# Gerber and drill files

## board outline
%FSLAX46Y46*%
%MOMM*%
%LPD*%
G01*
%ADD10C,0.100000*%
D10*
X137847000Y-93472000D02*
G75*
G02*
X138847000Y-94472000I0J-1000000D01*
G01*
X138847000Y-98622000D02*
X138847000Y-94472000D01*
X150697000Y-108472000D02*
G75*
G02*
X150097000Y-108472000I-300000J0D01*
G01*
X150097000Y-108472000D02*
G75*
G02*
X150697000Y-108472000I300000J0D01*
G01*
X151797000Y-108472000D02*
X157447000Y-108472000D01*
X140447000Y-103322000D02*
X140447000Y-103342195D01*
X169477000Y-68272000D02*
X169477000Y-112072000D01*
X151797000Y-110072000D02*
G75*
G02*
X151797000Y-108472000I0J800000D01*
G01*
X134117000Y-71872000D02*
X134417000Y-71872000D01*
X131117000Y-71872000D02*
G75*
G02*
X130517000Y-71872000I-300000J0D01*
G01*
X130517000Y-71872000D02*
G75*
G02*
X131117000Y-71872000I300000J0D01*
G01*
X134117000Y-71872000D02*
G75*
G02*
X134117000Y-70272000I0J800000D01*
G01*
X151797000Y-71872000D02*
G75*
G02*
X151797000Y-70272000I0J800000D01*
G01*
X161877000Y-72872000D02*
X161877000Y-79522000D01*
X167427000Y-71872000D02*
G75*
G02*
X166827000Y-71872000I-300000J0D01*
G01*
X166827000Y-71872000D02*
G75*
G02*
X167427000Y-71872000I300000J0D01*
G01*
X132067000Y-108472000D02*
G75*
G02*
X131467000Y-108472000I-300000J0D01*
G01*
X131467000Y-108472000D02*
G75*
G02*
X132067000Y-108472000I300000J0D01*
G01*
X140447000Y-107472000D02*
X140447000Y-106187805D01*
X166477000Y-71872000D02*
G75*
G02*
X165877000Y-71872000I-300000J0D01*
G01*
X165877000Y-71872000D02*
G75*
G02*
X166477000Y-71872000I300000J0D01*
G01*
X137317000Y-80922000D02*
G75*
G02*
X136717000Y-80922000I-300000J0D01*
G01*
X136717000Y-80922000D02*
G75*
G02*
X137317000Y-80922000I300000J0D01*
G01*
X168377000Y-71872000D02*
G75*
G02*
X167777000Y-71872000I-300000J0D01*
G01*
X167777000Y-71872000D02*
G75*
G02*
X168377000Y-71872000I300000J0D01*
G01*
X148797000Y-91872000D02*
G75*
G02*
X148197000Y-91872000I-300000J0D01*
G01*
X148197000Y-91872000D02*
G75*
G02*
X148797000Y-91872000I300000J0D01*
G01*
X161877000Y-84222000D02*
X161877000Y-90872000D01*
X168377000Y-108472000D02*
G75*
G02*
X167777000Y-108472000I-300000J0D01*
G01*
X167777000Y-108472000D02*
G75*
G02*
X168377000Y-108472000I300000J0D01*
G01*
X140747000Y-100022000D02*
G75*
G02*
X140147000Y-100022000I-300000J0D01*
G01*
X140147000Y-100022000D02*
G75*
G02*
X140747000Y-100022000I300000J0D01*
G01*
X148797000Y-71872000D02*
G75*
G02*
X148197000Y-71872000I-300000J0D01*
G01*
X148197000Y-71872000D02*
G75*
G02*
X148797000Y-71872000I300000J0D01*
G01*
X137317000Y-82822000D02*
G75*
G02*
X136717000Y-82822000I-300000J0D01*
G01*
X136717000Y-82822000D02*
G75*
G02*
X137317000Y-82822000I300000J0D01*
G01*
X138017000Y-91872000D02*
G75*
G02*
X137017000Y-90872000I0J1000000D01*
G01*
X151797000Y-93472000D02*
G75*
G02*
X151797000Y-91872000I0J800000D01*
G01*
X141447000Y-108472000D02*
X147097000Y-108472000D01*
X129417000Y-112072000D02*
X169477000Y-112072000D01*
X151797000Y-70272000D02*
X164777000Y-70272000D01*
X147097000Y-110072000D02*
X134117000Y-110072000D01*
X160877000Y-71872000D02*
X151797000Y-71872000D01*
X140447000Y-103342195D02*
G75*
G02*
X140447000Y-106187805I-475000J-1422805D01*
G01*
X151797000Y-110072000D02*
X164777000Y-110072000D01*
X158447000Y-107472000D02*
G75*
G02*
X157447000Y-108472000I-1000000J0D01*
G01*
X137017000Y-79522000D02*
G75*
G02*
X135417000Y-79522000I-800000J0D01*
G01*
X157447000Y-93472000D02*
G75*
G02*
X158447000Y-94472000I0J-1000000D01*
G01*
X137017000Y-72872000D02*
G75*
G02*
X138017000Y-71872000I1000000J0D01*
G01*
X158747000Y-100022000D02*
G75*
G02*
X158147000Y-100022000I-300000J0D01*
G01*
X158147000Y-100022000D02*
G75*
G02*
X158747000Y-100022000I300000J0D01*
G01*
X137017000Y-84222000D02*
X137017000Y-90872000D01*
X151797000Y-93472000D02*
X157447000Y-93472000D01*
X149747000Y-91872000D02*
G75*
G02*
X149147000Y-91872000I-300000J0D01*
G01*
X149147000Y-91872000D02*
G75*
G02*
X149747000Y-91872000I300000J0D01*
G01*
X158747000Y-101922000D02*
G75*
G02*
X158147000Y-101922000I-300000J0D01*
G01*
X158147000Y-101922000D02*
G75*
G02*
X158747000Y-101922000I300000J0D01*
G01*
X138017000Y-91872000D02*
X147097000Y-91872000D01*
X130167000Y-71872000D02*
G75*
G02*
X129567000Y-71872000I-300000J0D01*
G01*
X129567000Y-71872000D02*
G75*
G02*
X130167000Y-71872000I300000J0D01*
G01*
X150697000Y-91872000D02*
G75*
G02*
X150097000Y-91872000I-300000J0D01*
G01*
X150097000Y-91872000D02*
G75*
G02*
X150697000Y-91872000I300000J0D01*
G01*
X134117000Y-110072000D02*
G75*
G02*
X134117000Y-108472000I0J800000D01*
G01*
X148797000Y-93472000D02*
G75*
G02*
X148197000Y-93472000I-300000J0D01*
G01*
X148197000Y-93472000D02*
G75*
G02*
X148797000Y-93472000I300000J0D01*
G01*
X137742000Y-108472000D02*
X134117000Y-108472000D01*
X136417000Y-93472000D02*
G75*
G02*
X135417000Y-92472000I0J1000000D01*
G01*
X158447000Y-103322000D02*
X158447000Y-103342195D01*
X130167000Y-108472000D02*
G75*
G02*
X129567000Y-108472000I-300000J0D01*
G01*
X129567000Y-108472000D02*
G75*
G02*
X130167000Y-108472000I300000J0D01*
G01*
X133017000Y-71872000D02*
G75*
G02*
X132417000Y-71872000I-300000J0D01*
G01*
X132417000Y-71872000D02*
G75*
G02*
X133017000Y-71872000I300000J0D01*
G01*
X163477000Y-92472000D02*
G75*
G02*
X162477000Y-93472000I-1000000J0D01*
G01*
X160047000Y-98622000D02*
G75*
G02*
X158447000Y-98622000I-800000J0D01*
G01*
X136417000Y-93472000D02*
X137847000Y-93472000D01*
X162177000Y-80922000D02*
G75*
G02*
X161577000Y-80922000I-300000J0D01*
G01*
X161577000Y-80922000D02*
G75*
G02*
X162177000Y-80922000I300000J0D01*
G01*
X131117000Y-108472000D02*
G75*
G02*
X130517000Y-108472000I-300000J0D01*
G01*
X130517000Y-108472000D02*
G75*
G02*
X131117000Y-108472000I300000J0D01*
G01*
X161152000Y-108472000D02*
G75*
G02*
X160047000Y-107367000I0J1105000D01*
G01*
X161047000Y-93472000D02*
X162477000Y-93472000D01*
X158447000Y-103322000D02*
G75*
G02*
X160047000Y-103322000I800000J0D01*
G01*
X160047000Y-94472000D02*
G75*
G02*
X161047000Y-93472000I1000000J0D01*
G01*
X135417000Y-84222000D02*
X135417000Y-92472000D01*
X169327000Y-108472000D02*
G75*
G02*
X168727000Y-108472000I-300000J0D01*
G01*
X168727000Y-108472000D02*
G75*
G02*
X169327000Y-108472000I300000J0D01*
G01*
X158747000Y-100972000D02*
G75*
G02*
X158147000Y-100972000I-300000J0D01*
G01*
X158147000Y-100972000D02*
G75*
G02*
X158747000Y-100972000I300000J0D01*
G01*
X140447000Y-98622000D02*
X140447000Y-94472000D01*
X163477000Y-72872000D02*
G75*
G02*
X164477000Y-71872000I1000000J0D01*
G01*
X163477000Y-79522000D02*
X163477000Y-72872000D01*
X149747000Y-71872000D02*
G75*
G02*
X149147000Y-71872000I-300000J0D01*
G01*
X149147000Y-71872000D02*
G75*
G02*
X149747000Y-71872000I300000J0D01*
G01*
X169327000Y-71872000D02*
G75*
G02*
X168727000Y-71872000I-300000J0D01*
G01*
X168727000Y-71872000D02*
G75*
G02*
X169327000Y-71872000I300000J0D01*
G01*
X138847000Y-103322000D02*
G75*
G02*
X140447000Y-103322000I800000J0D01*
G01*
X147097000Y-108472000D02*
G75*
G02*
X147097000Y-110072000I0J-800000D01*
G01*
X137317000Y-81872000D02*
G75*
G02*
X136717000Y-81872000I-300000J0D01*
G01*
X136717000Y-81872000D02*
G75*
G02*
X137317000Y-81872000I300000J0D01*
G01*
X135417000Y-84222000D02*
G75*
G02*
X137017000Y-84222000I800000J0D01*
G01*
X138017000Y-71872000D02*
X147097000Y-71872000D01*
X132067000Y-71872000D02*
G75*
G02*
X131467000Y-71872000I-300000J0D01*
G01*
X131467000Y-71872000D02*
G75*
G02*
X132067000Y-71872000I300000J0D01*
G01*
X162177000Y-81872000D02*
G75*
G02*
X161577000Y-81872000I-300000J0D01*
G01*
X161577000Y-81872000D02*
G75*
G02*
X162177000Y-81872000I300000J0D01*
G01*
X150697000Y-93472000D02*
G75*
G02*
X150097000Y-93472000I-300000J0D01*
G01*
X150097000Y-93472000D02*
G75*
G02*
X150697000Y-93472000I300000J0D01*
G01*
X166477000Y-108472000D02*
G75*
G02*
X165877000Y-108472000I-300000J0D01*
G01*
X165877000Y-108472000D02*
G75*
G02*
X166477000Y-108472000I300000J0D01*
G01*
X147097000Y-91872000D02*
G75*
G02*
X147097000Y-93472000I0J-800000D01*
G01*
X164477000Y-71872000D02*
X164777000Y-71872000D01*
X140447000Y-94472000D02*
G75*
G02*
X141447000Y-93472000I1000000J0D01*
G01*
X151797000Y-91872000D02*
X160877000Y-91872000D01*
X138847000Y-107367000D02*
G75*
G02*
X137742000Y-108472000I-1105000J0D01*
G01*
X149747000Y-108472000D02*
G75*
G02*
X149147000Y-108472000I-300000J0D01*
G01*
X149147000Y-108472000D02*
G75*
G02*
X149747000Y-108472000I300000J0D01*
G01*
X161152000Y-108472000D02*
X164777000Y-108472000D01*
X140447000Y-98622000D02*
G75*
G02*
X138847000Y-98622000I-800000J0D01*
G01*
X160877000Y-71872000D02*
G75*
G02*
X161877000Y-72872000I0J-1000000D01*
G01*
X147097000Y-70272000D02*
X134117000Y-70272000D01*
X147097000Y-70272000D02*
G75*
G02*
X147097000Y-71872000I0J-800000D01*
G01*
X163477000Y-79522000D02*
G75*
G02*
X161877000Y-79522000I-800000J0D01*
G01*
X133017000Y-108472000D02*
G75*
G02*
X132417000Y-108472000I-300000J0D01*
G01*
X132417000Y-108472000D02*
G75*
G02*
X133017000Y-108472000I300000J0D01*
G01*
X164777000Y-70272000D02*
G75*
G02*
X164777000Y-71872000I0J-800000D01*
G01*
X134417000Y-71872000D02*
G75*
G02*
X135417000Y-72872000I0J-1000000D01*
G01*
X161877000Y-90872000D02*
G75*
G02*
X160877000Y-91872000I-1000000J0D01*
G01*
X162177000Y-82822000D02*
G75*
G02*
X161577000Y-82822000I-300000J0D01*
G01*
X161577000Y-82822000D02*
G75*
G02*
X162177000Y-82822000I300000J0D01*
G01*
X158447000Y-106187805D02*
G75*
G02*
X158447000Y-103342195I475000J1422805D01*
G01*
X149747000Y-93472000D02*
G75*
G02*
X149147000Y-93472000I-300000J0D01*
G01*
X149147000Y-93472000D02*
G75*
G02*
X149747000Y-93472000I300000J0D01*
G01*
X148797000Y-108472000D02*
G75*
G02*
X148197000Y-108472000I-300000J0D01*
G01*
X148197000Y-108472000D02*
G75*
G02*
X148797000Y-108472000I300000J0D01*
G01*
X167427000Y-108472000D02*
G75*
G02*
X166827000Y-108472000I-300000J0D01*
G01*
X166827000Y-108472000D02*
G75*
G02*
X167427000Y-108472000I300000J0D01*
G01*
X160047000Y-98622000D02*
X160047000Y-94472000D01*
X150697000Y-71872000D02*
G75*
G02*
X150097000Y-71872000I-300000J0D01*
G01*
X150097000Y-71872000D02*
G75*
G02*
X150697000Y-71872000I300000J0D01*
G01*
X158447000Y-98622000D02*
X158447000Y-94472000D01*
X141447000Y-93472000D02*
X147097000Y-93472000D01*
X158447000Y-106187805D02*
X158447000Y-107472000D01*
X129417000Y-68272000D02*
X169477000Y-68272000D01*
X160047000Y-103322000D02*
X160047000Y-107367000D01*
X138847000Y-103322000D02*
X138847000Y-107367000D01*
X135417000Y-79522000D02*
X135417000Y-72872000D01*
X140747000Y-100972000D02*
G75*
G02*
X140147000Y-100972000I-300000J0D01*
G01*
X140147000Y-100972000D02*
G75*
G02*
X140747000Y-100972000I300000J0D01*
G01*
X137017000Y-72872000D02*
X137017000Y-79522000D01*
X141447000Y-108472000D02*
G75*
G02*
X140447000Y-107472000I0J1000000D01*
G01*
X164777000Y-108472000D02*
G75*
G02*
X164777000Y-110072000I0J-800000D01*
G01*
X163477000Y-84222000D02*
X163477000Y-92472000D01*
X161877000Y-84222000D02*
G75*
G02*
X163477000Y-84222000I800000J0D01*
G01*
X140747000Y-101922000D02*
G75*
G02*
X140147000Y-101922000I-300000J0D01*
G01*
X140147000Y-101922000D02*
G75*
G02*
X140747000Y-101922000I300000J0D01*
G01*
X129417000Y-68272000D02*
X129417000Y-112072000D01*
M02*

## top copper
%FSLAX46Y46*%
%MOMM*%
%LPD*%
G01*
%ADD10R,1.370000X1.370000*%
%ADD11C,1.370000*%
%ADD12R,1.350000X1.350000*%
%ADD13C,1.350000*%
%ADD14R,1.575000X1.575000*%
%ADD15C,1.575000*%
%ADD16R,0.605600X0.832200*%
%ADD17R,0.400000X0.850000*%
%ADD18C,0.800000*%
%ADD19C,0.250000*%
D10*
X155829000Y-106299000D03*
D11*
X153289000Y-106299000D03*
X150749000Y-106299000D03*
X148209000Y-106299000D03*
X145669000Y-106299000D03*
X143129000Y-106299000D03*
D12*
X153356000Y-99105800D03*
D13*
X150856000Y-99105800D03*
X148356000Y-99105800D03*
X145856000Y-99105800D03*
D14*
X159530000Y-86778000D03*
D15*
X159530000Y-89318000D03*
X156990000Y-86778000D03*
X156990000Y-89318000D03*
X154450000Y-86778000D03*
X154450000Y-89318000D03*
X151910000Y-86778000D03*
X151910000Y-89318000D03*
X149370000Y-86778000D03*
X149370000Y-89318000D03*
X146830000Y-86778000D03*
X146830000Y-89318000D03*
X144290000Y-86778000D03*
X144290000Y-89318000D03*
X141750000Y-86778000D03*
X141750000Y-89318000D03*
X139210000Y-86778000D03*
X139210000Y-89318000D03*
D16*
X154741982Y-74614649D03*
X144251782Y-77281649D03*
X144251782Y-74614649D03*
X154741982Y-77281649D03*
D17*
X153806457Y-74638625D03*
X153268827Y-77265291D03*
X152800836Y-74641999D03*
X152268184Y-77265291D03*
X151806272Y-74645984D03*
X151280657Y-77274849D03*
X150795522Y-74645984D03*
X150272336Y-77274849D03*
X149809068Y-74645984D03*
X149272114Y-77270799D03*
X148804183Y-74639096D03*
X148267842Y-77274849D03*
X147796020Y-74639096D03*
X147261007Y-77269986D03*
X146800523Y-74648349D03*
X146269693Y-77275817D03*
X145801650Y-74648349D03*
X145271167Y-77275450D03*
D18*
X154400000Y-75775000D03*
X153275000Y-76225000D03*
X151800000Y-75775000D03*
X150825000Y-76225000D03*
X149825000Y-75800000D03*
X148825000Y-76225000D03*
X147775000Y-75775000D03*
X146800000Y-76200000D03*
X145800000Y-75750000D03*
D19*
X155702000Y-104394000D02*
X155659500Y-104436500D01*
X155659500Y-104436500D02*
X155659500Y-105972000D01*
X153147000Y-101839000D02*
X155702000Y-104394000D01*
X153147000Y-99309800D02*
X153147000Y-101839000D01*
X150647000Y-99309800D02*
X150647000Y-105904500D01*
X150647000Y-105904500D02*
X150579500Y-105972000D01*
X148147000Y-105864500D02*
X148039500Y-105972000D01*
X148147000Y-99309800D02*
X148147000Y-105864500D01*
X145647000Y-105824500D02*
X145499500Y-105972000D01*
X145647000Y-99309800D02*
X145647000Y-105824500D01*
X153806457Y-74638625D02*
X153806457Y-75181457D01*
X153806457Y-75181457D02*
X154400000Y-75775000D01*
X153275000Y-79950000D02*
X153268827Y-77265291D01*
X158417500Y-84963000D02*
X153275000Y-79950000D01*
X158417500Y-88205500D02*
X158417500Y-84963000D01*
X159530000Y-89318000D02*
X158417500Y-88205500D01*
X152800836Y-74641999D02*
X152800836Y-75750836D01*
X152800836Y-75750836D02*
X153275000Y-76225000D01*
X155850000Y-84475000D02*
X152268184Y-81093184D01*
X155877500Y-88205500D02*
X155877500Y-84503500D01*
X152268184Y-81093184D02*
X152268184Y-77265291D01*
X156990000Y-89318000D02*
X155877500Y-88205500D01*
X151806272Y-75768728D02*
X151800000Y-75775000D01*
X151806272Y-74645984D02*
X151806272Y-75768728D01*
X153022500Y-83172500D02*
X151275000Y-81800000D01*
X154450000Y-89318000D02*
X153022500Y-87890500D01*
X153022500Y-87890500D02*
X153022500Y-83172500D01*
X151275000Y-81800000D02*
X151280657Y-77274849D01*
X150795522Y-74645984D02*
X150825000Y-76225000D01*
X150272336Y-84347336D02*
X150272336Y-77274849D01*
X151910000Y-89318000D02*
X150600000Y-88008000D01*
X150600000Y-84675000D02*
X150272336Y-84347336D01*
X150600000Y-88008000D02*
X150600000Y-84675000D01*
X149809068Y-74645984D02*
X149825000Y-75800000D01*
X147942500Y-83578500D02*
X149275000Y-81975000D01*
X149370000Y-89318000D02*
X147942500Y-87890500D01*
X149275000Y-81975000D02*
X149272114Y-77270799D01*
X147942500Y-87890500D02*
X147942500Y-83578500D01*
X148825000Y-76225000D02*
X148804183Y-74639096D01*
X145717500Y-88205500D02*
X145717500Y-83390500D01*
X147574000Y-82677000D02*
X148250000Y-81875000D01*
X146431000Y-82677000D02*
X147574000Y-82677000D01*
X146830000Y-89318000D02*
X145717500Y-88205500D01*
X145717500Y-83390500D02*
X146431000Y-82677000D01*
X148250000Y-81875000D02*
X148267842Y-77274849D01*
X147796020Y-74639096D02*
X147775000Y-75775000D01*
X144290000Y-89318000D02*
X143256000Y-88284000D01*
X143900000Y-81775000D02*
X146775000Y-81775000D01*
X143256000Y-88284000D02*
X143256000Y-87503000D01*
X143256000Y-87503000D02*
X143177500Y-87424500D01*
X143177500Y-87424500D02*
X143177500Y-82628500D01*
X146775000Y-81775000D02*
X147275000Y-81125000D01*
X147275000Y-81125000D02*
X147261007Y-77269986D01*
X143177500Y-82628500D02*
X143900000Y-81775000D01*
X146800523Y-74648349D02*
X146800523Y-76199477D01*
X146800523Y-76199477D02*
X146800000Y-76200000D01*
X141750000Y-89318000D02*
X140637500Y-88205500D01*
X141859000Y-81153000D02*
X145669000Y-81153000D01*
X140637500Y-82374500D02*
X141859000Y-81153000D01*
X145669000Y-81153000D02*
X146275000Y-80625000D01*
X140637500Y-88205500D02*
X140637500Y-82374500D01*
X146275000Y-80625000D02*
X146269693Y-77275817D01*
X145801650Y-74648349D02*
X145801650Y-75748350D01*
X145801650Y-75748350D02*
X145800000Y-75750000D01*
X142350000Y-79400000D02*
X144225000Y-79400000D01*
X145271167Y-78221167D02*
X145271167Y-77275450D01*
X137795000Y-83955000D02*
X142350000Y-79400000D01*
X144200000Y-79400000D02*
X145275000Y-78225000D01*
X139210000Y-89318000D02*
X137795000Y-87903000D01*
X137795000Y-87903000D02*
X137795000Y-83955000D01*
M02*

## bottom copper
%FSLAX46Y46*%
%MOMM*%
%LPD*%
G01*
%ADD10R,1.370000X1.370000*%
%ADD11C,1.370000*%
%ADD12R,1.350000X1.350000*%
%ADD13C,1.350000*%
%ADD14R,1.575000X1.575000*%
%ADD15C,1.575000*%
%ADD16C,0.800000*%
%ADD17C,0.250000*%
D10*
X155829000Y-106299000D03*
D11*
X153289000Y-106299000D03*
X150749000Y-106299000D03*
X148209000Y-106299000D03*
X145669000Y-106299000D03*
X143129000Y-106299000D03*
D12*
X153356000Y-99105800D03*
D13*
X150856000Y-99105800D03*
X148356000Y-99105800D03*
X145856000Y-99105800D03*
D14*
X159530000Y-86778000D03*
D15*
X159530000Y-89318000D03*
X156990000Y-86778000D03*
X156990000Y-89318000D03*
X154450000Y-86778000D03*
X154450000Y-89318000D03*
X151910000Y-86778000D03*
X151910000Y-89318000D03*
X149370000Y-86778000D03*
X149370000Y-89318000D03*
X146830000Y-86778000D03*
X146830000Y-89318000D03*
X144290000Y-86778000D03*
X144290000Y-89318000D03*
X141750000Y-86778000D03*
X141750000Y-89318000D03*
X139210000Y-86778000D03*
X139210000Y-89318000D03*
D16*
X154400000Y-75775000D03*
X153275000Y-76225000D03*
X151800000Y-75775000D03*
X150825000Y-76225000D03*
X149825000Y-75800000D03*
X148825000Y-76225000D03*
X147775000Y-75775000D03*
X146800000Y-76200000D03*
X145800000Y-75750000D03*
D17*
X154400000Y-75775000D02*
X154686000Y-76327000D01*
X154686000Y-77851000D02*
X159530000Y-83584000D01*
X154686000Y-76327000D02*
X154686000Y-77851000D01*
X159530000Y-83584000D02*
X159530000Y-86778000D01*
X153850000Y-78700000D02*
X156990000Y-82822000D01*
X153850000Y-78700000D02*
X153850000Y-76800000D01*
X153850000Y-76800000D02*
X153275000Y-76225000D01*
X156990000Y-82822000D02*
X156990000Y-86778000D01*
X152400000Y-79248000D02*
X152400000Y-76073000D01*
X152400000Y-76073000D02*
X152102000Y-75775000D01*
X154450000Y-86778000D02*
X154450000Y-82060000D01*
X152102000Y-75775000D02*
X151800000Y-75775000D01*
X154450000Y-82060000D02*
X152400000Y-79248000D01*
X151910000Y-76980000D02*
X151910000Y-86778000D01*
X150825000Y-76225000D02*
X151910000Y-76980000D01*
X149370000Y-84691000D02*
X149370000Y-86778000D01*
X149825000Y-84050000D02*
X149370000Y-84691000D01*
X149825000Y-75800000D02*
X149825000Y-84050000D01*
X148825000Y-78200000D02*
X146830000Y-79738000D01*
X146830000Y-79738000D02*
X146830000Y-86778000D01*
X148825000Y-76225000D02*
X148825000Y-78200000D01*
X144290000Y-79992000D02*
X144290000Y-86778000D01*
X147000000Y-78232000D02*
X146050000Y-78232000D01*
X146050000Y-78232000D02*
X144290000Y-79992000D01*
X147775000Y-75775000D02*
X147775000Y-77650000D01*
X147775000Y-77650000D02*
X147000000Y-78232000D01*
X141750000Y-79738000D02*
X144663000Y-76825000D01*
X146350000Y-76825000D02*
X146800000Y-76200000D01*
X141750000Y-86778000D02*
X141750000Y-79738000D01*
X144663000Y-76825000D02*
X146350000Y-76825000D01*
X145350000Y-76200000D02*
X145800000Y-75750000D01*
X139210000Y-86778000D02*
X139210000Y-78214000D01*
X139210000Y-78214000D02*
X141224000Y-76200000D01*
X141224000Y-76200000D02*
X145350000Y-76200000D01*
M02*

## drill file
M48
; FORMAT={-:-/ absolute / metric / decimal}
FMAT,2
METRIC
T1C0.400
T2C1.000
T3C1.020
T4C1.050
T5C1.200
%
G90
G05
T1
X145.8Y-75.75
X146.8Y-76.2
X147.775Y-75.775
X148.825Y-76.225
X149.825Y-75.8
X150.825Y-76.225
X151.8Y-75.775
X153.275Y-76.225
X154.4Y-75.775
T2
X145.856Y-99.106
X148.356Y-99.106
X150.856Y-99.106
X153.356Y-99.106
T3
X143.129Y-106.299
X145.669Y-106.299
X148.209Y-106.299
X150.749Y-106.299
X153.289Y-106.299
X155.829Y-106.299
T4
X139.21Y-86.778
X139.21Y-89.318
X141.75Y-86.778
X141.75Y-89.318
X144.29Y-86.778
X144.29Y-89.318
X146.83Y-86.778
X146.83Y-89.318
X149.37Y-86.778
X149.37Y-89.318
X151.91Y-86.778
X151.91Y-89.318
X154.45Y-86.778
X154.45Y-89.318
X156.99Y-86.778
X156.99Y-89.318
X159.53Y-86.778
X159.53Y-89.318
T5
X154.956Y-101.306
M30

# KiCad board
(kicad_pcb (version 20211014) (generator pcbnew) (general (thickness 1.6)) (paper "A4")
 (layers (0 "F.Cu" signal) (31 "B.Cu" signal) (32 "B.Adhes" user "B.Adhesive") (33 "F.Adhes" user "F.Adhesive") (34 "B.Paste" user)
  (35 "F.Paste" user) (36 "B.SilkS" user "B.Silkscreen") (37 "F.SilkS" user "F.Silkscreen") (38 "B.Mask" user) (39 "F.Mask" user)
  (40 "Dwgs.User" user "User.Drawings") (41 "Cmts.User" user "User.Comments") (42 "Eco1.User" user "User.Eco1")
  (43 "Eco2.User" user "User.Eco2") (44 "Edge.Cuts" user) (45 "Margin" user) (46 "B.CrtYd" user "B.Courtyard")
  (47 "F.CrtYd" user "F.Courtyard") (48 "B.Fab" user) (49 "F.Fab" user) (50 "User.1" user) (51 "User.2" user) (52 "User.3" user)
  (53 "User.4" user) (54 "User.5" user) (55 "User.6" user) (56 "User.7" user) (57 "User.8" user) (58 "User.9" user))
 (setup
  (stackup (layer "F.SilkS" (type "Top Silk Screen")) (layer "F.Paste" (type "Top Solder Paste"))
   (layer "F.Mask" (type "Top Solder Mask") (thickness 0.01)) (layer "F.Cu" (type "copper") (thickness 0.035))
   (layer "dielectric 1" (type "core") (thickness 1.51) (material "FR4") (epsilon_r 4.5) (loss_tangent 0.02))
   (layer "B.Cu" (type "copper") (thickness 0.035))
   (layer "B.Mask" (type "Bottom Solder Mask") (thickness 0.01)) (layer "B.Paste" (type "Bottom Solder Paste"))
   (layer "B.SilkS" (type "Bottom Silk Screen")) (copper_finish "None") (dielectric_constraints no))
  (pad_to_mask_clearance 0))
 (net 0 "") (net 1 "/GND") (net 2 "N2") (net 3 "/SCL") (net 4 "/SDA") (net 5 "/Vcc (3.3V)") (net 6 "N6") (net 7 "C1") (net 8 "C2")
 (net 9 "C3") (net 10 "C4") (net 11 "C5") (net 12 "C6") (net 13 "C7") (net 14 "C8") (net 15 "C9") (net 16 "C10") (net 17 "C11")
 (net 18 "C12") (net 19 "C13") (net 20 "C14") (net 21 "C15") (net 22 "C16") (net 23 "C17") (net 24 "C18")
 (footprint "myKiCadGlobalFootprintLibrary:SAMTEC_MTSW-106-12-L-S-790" (layer "F.Cu") (at 149.479 106.299)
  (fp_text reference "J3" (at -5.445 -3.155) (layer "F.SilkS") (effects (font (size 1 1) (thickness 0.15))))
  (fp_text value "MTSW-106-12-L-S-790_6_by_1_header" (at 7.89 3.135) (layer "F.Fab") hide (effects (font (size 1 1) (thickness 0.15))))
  (pad "01" thru_hole rect (at 6.35 0) (size 1.37 1.37) (drill 1.02) (layers *.Cu *.Mask) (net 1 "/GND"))
  (pad "02" thru_hole circle (at 3.81 0) (size 1.37 1.37) (drill 1.02) (layers *.Cu *.Mask) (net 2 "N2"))
  (pad "03" thru_hole circle (at 1.27 0) (size 1.37 1.37) (drill 1.02) (layers *.Cu *.Mask) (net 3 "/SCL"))
  (pad "04" thru_hole circle (at -1.27 0) (size 1.37 1.37) (drill 1.02) (layers *.Cu *.Mask) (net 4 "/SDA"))
  (pad "05" thru_hole circle (at -3.81 0) (size 1.37 1.37) (drill 1.02) (layers *.Cu *.Mask) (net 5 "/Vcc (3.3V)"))
  (pad "06" thru_hole circle (at -6.35 0) (size 1.37 1.37) (drill 1.02) (layers *.Cu *.Mask) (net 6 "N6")))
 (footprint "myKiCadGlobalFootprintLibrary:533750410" (layer "F.Cu") (at 153.356 99.1058)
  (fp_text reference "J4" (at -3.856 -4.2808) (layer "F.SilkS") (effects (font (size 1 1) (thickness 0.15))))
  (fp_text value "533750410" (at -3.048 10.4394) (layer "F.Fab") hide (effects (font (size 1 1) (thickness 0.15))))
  (pad "" np_thru_hole circle (at 1.6 2.2) (size 1.2 1.2) (drill 1.2) (layers *.Cu *.Mask))
  (pad "1" thru_hole rect (at 0 0) (size 1.35 1.35) (drill 1) (layers *.Cu) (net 1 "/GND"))
  (pad "2" thru_hole circle (at -2.5 0) (size 1.35 1.35) (drill 1) (layers *.Cu) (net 3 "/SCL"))
  (pad "3" thru_hole circle (at -5 0) (size 1.35 1.35) (drill 1) (layers *.Cu) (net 4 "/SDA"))
  (pad "4" thru_hole circle (at -7.5 0) (size 1.35 1.35) (drill 1) (layers *.Cu) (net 5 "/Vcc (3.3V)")))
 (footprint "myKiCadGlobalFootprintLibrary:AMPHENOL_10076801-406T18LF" (layer "F.Cu") (at 149.37 88.048 180)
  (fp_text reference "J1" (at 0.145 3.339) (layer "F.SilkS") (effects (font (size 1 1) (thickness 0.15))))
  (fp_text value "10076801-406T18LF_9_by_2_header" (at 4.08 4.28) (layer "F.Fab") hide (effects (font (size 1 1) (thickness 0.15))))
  (pad "01" thru_hole rect (at -10.16 1.27 180) (size 1.575 1.575) (drill 1.05) (layers *.Cu *.Mask) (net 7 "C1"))
  (pad "02" thru_hole circle (at -10.16 -1.27 180) (size 1.575 1.575) (drill 1.05) (layers *.Cu *.Mask) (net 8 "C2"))
  (pad "03" thru_hole circle (at -7.62 1.27 180) (size 1.575 1.575) (drill 1.05) (layers *.Cu *.Mask) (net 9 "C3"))
  (pad "04" thru_hole circle (at -7.62 -1.27 180) (size 1.575 1.575) (drill 1.05) (layers *.Cu *.Mask) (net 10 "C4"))
  (pad "05" thru_hole circle (at -5.08 1.27 180) (size 1.575 1.575) (drill 1.05) (layers *.Cu *.Mask) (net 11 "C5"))
  (pad "06" thru_hole circle (at -5.08 -1.27 180) (size 1.575 1.575) (drill 1.05) (layers *.Cu *.Mask) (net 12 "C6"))
  (pad "07" thru_hole circle (at -2.54 1.27 180) (size 1.575 1.575) (drill 1.05) (layers *.Cu *.Mask) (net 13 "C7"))
  (pad "08" thru_hole circle (at -2.54 -1.27 180) (size 1.575 1.575) (drill 1.05) (layers *.Cu *.Mask) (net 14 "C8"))
  (pad "09" thru_hole circle (at 0 1.27 180) (size 1.575 1.575) (drill 1.05) (layers *.Cu *.Mask) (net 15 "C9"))
  (pad "10" thru_hole circle (at 0 -1.27 180) (size 1.575 1.575) (drill 1.05) (layers *.Cu *.Mask) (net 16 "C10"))
  (pad "11" thru_hole circle (at 2.54 1.27 180) (size 1.575 1.575) (drill 1.05) (layers *.Cu *.Mask) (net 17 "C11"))
  (pad "12" thru_hole circle (at 2.54 -1.27 180) (size 1.575 1.575) (drill 1.05) (layers *.Cu *.Mask) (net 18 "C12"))
  (pad "13" thru_hole circle (at 5.08 1.27 180) (size 1.575 1.575) (drill 1.05) (layers *.Cu *.Mask) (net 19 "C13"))
  (pad "14" thru_hole circle (at 5.08 -1.27 180) (size 1.575 1.575) (drill 1.05) (layers *.Cu *.Mask) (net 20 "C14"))
  (pad "15" thru_hole circle (at 7.62 1.27 180) (size 1.575 1.575) (drill 1.05) (layers *.Cu *.Mask) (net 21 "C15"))
  (pad "16" thru_hole circle (at 7.62 -1.27 180) (size 1.575 1.575) (drill 1.05) (layers *.Cu *.Mask) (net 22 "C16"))
  (pad "17" thru_hole circle (at 10.16 1.27 180) (size 1.575 1.575) (drill 1.05) (layers *.Cu *.Mask) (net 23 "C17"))
  (pad "18" thru_hole circle (at 10.16 -1.27 180) (size 1.575 1.575) (drill 1.05) (layers *.Cu *.Mask) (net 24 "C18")))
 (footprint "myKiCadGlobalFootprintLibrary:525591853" (layer "F.Cu") (at 149.280982 75.605249)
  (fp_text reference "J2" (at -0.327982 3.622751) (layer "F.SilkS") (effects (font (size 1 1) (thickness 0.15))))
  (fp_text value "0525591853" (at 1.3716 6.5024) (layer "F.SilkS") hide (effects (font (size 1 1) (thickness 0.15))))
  (pad " " smd rect (at 5.461 -0.9906) (size 0.6056 0.8322) (layers "F.Cu" "F.Paste" "F.Mask"))
  (pad " " smd rect (at -5.0292 1.6764) (size 0.6056 0.8322) (layers "F.Cu" "F.Paste" "F.Mask"))
  (pad " " smd rect (at -5.0292 -0.9906) (size 0.6056 0.8322) (layers "F.Cu" "F.Paste" "F.Mask"))
  (pad " " smd rect (at 5.461 1.6764) (size 0.6056 0.8322) (layers "F.Cu" "F.Paste" "F.Mask"))
  (pad "1" smd rect (at 4.525475 -0.966624) (size 0.4 0.85) (layers "F.Cu" "F.Paste" "F.Mask") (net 7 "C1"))
  (pad "2" smd rect (at 3.987845 1.660042) (size 0.4 0.85) (layers "F.Cu" "F.Paste" "F.Mask") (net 8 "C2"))
  (pad "3" smd rect (at 3.519854 -0.96325) (size 0.4 0.85) (layers "F.Cu" "F.Paste" "F.Mask") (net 9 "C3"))
  (pad "4" smd rect (at 2.987202 1.660042) (size 0.4 0.85) (layers "F.Cu" "F.Paste" "F.Mask") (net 10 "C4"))
  (pad "5" smd rect (at 2.52529 -0.959265) (size 0.4 0.85) (layers "F.Cu" "F.Paste" "F.Mask") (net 11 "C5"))
  (pad "6" smd rect (at 1.999675 1.6696) (size 0.4 0.85) (layers "F.Cu" "F.Paste" "F.Mask") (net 12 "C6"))
  (pad "7" smd rect (at 1.51454 -0.959265) (size 0.4 0.85) (layers "F.Cu" "F.Paste" "F.Mask") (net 13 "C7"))
  (pad "8" smd rect (at 0.991354 1.6696) (size 0.4 0.85) (layers "F.Cu" "F.Paste" "F.Mask") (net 14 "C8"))
  (pad "9" smd rect (at 0.528086 -0.959265) (size 0.4 0.85) (layers "F.Cu" "F.Paste" "F.Mask") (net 15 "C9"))
  (pad "10" smd rect (at -0.008868 1.66555) (size 0.4 0.85) (layers "F.Cu" "F.Paste" "F.Mask") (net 16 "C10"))
  (pad "11" smd rect (at -0.476799 -0.966153) (size 0.4 0.85) (layers "F.Cu" "F.Paste" "F.Mask") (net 17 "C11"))
  (pad "12" smd rect (at -1.01314 1.6696) (size 0.4 0.85) (layers "F.Cu" "F.Paste" "F.Mask") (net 18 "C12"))
  (pad "13" smd rect (at -1.484962 -0.966153) (size 0.4 0.85) (layers "F.Cu" "F.Paste" "F.Mask") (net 19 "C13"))
  (pad "14" smd rect (at -2.019975 1.664737) (size 0.4 0.85) (layers "F.Cu" "F.Paste" "F.Mask") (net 20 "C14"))
  (pad "15" smd rect (at -2.480459 -0.9569) (size 0.4 0.85) (layers "F.Cu" "F.Paste" "F.Mask") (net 21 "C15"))
  (pad "16" smd rect (at -3.011289 1.670568) (size 0.4 0.85) (layers "F.Cu" "F.Paste" "F.Mask") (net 22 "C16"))
  (pad "17" smd rect (at -3.479332 -0.9569) (size 0.4 0.85) (layers "F.Cu" "F.Paste" "F.Mask") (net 23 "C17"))
  (pad "18" smd rect (at -4.009815 1.670201) (size 0.4 0.85) (layers "F.Cu" "F.Paste" "F.Mask") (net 24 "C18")))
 (gr_arc (start 137.847 93.472) (mid 138.554107 93.764893) (end 138.847 94.472) (layer "Edge.Cuts") (width 0.1))
 (gr_line (start 138.847 98.622) (end 138.847 94.472) (layer "Edge.Cuts") (width 0.1))
 (gr_circle (center 150.397 108.472) (end 150.697 108.472) (layer "Edge.Cuts") (width 0.1) (fill none))
 (gr_line (start 151.797 108.472) (end 157.447 108.472) (layer "Edge.Cuts") (width 0.1))
 (gr_line (start 140.447 103.322) (end 140.447 103.342195) (layer "Edge.Cuts") (width 0.1))
 (gr_line (start 169.477 68.272) (end 169.477 112.072) (layer "Edge.Cuts") (width 0.1))
 (gr_arc (start 151.797 110.072) (mid 150.997 109.272) (end 151.797 108.472) (layer "Edge.Cuts") (width 0.1))
 (gr_line (start 134.117 71.872) (end 134.417 71.872) (layer "Edge.Cuts") (width 0.1))
 (gr_circle (center 130.817 71.872) (end 131.117 71.872) (layer "Edge.Cuts") (width 0.1) (fill none))
 (gr_arc (start 134.117 71.872) (mid 133.317 71.072) (end 134.117 70.272) (layer "Edge.Cuts") (width 0.1))
 (gr_arc (start 151.797 71.872) (mid 150.997 71.072) (end 151.797 70.272) (layer "Edge.Cuts") (width 0.1))
 (gr_line (start 161.877 72.872) (end 161.877 79.522) (layer "Edge.Cuts") (width 0.1))
 (gr_circle (center 167.127 71.872) (end 167.427 71.872) (layer "Edge.Cuts") (width 0.1) (fill none))
 (gr_circle (center 131.767 108.472) (end 132.067 108.472) (layer "Edge.Cuts") (width 0.1) (fill none))
 (gr_line (start 140.447 107.472) (end 140.447 106.187805) (layer "Edge.Cuts") (width 0.1))
 (gr_circle (center 166.177 71.872) (end 166.477 71.872) (layer "Edge.Cuts") (width 0.1) (fill none))
 (gr_circle (center 137.017 80.922) (end 137.317 80.922) (layer "Edge.Cuts") (width 0.1) (fill none))
 (gr_circle (center 168.077 71.872) (end 168.377 71.872) (layer "Edge.Cuts") (width 0.1) (fill none))
 (gr_circle (center 148.497 91.872) (end 148.797 91.872) (layer "Edge.Cuts") (width 0.1) (fill none))
 (gr_line (start 161.877 84.222) (end 161.877 90.872) (layer "Edge.Cuts") (width 0.1))
 (gr_circle (center 168.077 108.472) (end 168.377 108.472) (layer "Edge.Cuts") (width 0.1) (fill none))
 (gr_circle (center 140.447 100.022) (end 140.747 100.022) (layer "Edge.Cuts") (width 0.1) (fill none))
 (gr_circle (center 148.497 71.872) (end 148.797 71.872) (layer "Edge.Cuts") (width 0.1) (fill none))
 (gr_circle (center 137.017 82.822) (end 137.317 82.822) (layer "Edge.Cuts") (width 0.1) (fill none))
 (gr_arc (start 138.017 91.872) (mid 137.309893 91.579107) (end 137.017 90.872) (layer "Edge.Cuts") (width 0.1))
 (gr_arc (start 151.797 93.472) (mid 150.997 92.672) (end 151.797 91.872) (layer "Edge.Cuts") (width 0.1))
 (gr_line (start 141.447 108.472) (end 147.097 108.472) (layer "Edge.Cuts") (width 0.1))
 (gr_line (start 129.417 112.072) (end 169.477 112.072) (layer "Edge.Cuts") (width 0.1))
 (gr_line (start 151.797 70.272) (end 164.777 70.272) (layer "Edge.Cuts") (width 0.1))
 (gr_line (start 147.097 110.072) (end 134.117 110.072) (layer "Edge.Cuts") (width 0.1))
 (gr_line (start 160.877 71.872) (end 151.797 71.872) (layer "Edge.Cuts") (width 0.1))
 (gr_arc (start 140.447 103.342195) (mid 141.472 104.765) (end 140.447 106.187805) (layer "Edge.Cuts") (width 0.1))
 (gr_line (start 151.797 110.072) (end 164.777 110.072) (layer "Edge.Cuts") (width 0.1))
 (gr_arc (start 158.447 107.472) (mid 158.154107 108.179107) (end 157.447 108.472) (layer "Edge.Cuts") (width 0.1))
 (gr_arc (start 137.017 79.522) (mid 136.217 80.322) (end 135.417 79.522) (layer "Edge.Cuts") (width 0.1))
 (gr_arc (start 157.447 93.472) (mid 158.154107 93.764893) (end 158.447 94.472) (layer "Edge.Cuts") (width 0.1))
 (gr_arc (start 137.017 72.872) (mid 137.309893 72.164893) (end 138.017 71.872) (layer "Edge.Cuts") (width 0.1))
 (gr_circle (center 158.447 100.022) (end 158.747 100.022) (layer "Edge.Cuts") (width 0.1) (fill none))
 (gr_line (start 137.017 84.222) (end 137.017 90.872) (layer "Edge.Cuts") (width 0.1))
 (gr_line (start 151.797 93.472) (end 157.447 93.472) (layer "Edge.Cuts") (width 0.1))
 (gr_circle (center 149.447 91.872) (end 149.747 91.872) (layer "Edge.Cuts") (width 0.1) (fill none))
 (gr_circle (center 158.447 101.922) (end 158.747 101.922) (layer "Edge.Cuts") (width 0.1) (fill none))
 (gr_line (start 138.017 91.872) (end 147.097 91.872) (layer "Edge.Cuts") (width 0.1))
 (gr_circle (center 129.867 71.872) (end 130.167 71.872) (layer "Edge.Cuts") (width 0.1) (fill none))
 (gr_circle (center 150.397 91.872) (end 150.697 91.872) (layer "Edge.Cuts") (width 0.1) (fill none))
 (gr_arc (start 134.117 110.072) (mid 133.317 109.272) (end 134.117 108.472) (layer "Edge.Cuts") (width 0.1))
 (gr_circle (center 148.497 93.472) (end 148.797 93.472) (layer "Edge.Cuts") (width 0.1) (fill none))
 (gr_line (start 137.742 108.472) (end 134.117 108.472) (layer "Edge.Cuts") (width 0.1))
 (gr_arc (start 136.417 93.472) (mid 135.709893 93.179107) (end 135.417 92.472) (layer "Edge.Cuts") (width 0.1))
 (gr_line (start 158.447 103.322) (end 158.447 103.342195) (layer "Edge.Cuts") (width 0.1))
 (gr_circle (center 129.867 108.472) (end 130.167 108.472) (layer "Edge.Cuts") (width 0.1) (fill none))
 (gr_circle (center 132.717 71.872) (end 133.017 71.872) (layer "Edge.Cuts") (width 0.1) (fill none))
 (gr_arc (start 163.477 92.472) (mid 163.184107 93.179107) (end 162.477 93.472) (layer "Edge.Cuts") (width 0.1))
 (gr_arc (start 160.047 98.622) (mid 159.247 99.422) (end 158.447 98.622) (layer "Edge.Cuts") (width 0.1))
 (gr_line (start 136.417 93.472) (end 137.847 93.472) (layer "Edge.Cuts") (width 0.1))
 (gr_circle (center 161.877 80.922) (end 162.177 80.922) (layer "Edge.Cuts") (width 0.1) (fill none))
 (gr_circle (center 130.817 108.472) (end 131.117 108.472) (layer "Edge.Cuts") (width 0.1) (fill none))
 (gr_arc (start 161.152 108.472) (mid 160.370647 108.148353) (end 160.047 107.367) (layer "Edge.Cuts") (width 0.1))
 (gr_line (start 161.047 93.472) (end 162.477 93.472) (layer "Edge.Cuts") (width 0.1))
 (gr_arc (start 158.447 103.322) (mid 159.247 102.522) (end 160.047 103.322) (layer "Edge.Cuts") (width 0.1))
 (gr_arc (start 160.047 94.472) (mid 160.339893 93.764893) (end 161.047 93.472) (layer "Edge.Cuts") (width 0.1))
 (gr_line (start 135.417 84.222) (end 135.417 92.472) (layer "Edge.Cuts") (width 0.1))
 (gr_circle (center 169.027 108.472) (end 169.327 108.472) (layer "Edge.Cuts") (width 0.1) (fill none))
 (gr_circle (center 158.447 100.972) (end 158.747 100.972) (layer "Edge.Cuts") (width 0.1) (fill none))
 (gr_line (start 140.447 98.622) (end 140.447 94.472) (layer "Edge.Cuts") (width 0.1))
 (gr_arc (start 163.477 72.872) (mid 163.769893 72.164893) (end 164.477 71.872) (layer "Edge.Cuts") (width 0.1))
 (gr_line (start 163.477 79.522) (end 163.477 72.872) (layer "Edge.Cuts") (width 0.1))
 (gr_circle (center 149.447 71.872) (end 149.747 71.872) (layer "Edge.Cuts") (width 0.1) (fill none))
 (gr_circle (center 169.027 71.872) (end 169.327 71.872) (layer "Edge.Cuts") (width 0.1) (fill none))
 (gr_arc (start 138.847 103.322) (mid 139.647 102.522) (end 140.447 103.322) (layer "Edge.Cuts") (width 0.1))
 (gr_arc (start 147.097 108.472) (mid 147.897 109.272) (end 147.097 110.072) (layer "Edge.Cuts") (width 0.1))
 (gr_circle (center 137.017 81.872) (end 137.317 81.872) (layer "Edge.Cuts") (width 0.1) (fill none))
 (gr_arc (start 135.417 84.222) (mid 136.217 83.422) (end 137.017 84.222) (layer "Edge.Cuts") (width 0.1))
 (gr_line (start 138.017 71.872) (end 147.097 71.872) (layer "Edge.Cuts") (width 0.1))
 (gr_circle (center 131.767 71.872) (end 132.067 71.872) (layer "Edge.Cuts") (width 0.1) (fill none))
 (gr_circle (center 161.877 81.872) (end 162.177 81.872) (layer "Edge.Cuts") (width 0.1) (fill none))
 (gr_circle (center 150.397 93.472) (end 150.697 93.472) (layer "Edge.Cuts") (width 0.1) (fill none))
 (gr_circle (center 166.177 108.472) (end 166.477 108.472) (layer "Edge.Cuts") (width 0.1) (fill none))
 (gr_arc (start 147.097 91.872) (mid 147.897 92.672) (end 147.097 93.472) (layer "Edge.Cuts") (width 0.1))
 (gr_line (start 164.477 71.872) (end 164.777 71.872) (layer "Edge.Cuts") (width 0.1))
 (gr_arc (start 140.447 94.472) (mid 140.739893 93.764893) (end 141.447 93.472) (layer "Edge.Cuts") (width 0.1))
 (gr_line (start 151.797 91.872) (end 160.877 91.872) (layer "Edge.Cuts") (width 0.1))
 (gr_arc (start 138.847 107.367) (mid 138.523353 108.148353) (end 137.742 108.472) (layer "Edge.Cuts") (width 0.1))
 (gr_circle (center 149.447 108.472) (end 149.747 108.472) (layer "Edge.Cuts") (width 0.1) (fill none))
 (gr_line (start 161.152 108.472) (end 164.777 108.472) (layer "Edge.Cuts") (width 0.1))
 (gr_arc (start 140.447 98.622) (mid 139.647 99.422) (end 138.847 98.622) (layer "Edge.Cuts") (width 0.1))
 (gr_arc (start 160.877 71.872) (mid 161.584107 72.164893) (end 161.877 72.872) (layer "Edge.Cuts") (width 0.1))
 (gr_line (start 147.097 70.272) (end 134.117 70.272) (layer "Edge.Cuts") (width 0.1))
 (gr_arc (start 147.097 70.272) (mid 147.897 71.072) (end 147.097 71.872) (layer "Edge.Cuts") (width 0.1))
 (gr_arc (start 163.477 79.522) (mid 162.677 80.322) (end 161.877 79.522) (layer "Edge.Cuts") (width 0.1))
 (gr_circle (center 132.717 108.472) (end 133.017 108.472) (layer "Edge.Cuts") (width 0.1) (fill none))
 (gr_arc (start 164.777 70.272) (mid 165.577 71.072) (end 164.777 71.872) (layer "Edge.Cuts") (width 0.1))
 (gr_arc (start 134.417 71.872) (mid 135.124107 72.164893) (end 135.417 72.872) (layer "Edge.Cuts") (width 0.1))
 (gr_arc (start 161.877 90.872) (mid 161.584107 91.579107) (end 160.877 91.872) (layer "Edge.Cuts") (width 0.1))
 (gr_circle (center 161.877 82.822) (end 162.177 82.822) (layer "Edge.Cuts") (width 0.1) (fill none))
 (gr_arc (start 158.447 106.187805) (mid 157.422 104.765) (end 158.447 103.342195) (layer "Edge.Cuts") (width 0.1))
 (gr_circle (center 149.447 93.472) (end 149.747 93.472) (layer "Edge.Cuts") (width 0.1) (fill none))
 (gr_circle (center 148.497 108.472) (end 148.797 108.472) (layer "Edge.Cuts") (width 0.1) (fill none))
 (gr_circle (center 167.127 108.472) (end 167.427 108.472) (layer "Edge.Cuts") (width 0.1) (fill none))
 (gr_line (start 160.047 98.622) (end 160.047 94.472) (layer "Edge.Cuts") (width 0.1))
 (gr_circle (center 150.397 71.872) (end 150.697 71.872) (layer "Edge.Cuts") (width 0.1) (fill none))
 (gr_line (start 158.447 98.622) (end 158.447 94.472) (layer "Edge.Cuts") (width 0.1))
 (gr_line (start 141.447 93.472) (end 147.097 93.472) (layer "Edge.Cuts") (width 0.1))
 (gr_line (start 158.447 106.187805) (end 158.447 107.472) (layer "Edge.Cuts") (width 0.1))
 (gr_line (start 129.417 68.272) (end 169.477 68.272) (layer "Edge.Cuts") (width 0.1))
 (gr_line (start 160.047 103.322) (end 160.047 107.367) (layer "Edge.Cuts") (width 0.1))
 (gr_line (start 138.847 103.322) (end 138.847 107.367) (layer "Edge.Cuts") (width 0.1))
 (gr_line (start 135.417 79.522) (end 135.417 72.872) (layer "Edge.Cuts") (width 0.1))
 (gr_circle (center 140.447 100.972) (end 140.747 100.972) (layer "Edge.Cuts") (width 0.1) (fill none))
 (gr_line (start 137.017 72.872) (end 137.017 79.522) (layer "Edge.Cuts") (width 0.1))
 (gr_arc (start 141.447 108.472) (mid 140.739893 108.179107) (end 140.447 107.472) (layer "Edge.Cuts") (width 0.1))
 (gr_arc (start 164.777 108.472) (mid 165.577 109.272) (end 164.777 110.072) (layer "Edge.Cuts") (width 0.1))
 (gr_line (start 163.477 84.222) (end 163.477 92.472) (layer "Edge.Cuts") (width 0.1))
 (gr_arc (start 161.877 84.222) (mid 162.677 83.422) (end 163.477 84.222) (layer "Edge.Cuts") (width 0.1))
 (gr_circle (center 140.447 101.922) (end 140.747 101.922) (layer "Edge.Cuts") (width 0.1) (fill none))
 (gr_line (start 129.417 68.272) (end 129.417 112.072) (layer "Edge.Cuts") (width 0.1))
 (segment (start 155.702 104.394) (end 155.6595 104.4365) (width 0.25) (layer "F.Cu") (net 1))
 (segment (start 155.6595 104.4365) (end 155.6595 105.972) (width 0.25) (layer "F.Cu") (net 1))
 (segment (start 153.147 101.839) (end 155.702 104.394) (width 0.25) (layer "F.Cu") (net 1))
 (segment (start 153.147 99.3098) (end 153.147 101.839) (width 0.25) (layer "F.Cu") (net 1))
 (segment (start 150.647 99.3098) (end 150.647 105.9045) (width 0.25) (layer "F.Cu") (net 3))
 (segment (start 150.647 105.9045) (end 150.5795 105.972) (width 0.25) (layer "F.Cu") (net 3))
 (segment (start 148.147 105.8645) (end 148.0395 105.972) (width 0.25) (layer "F.Cu") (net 4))
 (segment (start 148.147 99.3098) (end 148.147 105.8645) (width 0.25) (layer "F.Cu") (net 4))
 (segment (start 145.647 105.8245) (end 145.4995 105.972) (width 0.25) (layer "F.Cu") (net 5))
 (segment (start 145.647 99.3098) (end 145.647 105.8245) (width 0.25) (layer "F.Cu") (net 5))
 (segment (start 153.806457 74.638625) (end 153.806457 75.181457) (width 0.25) (layer "F.Cu") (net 7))
 (segment (start 153.806457 75.181457) (end 154.4 75.775) (width 0.25) (layer "F.Cu") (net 7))
 (via (at 154.4 75.775) (size 0.8) (drill 0.4) (layers "F.Cu" "B.Cu") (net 7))
 (segment (start 154.4 75.775) (end 154.686 76.327) (width 0.25) (layer "B.Cu") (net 7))
 (segment (start 154.686 77.851) (end 159.53 83.584) (width 0.25) (layer "B.Cu") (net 7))
 (segment (start 154.686 76.327) (end 154.686 77.851) (width 0.25) (layer "B.Cu") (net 7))
 (segment (start 159.53 83.584) (end 159.53 86.778) (width 0.25) (layer "B.Cu") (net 7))
 (segment (start 153.275 79.95) (end 153.268827 77.265291) (width 0.25) (layer "F.Cu") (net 8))
 (segment (start 158.4175 84.963) (end 153.275 79.95) (width 0.25) (layer "F.Cu") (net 8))
 (segment (start 158.4175 88.2055) (end 158.4175 84.963) (width 0.25) (layer "F.Cu") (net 8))
 (segment (start 159.53 89.318) (end 158.4175 88.2055) (width 0.25) (layer "F.Cu") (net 8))
 (segment (start 152.800836 74.641999) (end 152.800836 75.750836) (width 0.25) (layer "F.Cu") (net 9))
 (segment (start 152.800836 75.750836) (end 153.275 76.225) (width 0.25) (layer "F.Cu") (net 9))
 (via (at 153.275 76.225) (size 0.8) (drill 0.4) (layers "F.Cu" "B.Cu") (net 9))
 (segment (start 153.85 78.7) (end 156.99 82.822) (width 0.25) (layer "B.Cu") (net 9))
 (segment (start 153.85 78.7) (end 153.85 76.8) (width 0.25) (layer "B.Cu") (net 9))
 (segment (start 153.85 76.8) (end 153.275 76.225) (width 0.25) (layer "B.Cu") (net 9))
 (segment (start 156.99 82.822) (end 156.99 86.778) (width 0.25) (layer "B.Cu") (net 9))
 (segment (start 155.85 84.475) (end 152.268184 81.093184) (width 0.25) (layer "F.Cu") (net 10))
 (segment (start 155.8775 88.2055) (end 155.8775 84.5035) (width 0.25) (layer "F.Cu") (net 10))
 (segment (start 152.268184 81.093184) (end 152.268184 77.265291) (width 0.25) (layer "F.Cu") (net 10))
 (segment (start 156.99 89.318) (end 155.8775 88.2055) (width 0.25) (layer "F.Cu") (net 10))
 (segment (start 151.806272 75.768728) (end 151.8 75.775) (width 0.25) (layer "F.Cu") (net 11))
 (segment (start 151.806272 74.645984) (end 151.806272 75.768728) (width 0.25) (layer "F.Cu") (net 11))
 (via (at 151.8 75.775) (size 0.8) (drill 0.4) (layers "F.Cu" "B.Cu") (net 11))
 (segment (start 152.4 79.248) (end 152.4 76.073) (width 0.25) (layer "B.Cu") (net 11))
 (segment (start 152.4 76.073) (end 152.102 75.775) (width 0.25) (layer "B.Cu") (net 11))
 (segment (start 154.45 86.778) (end 154.45 82.06) (width 0.25) (layer "B.Cu") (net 11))
 (segment (start 152.102 75.775) (end 151.8 75.775) (width 0.25) (layer "B.Cu") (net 11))
 (segment (start 154.45 82.06) (end 152.4 79.248) (width 0.25) (layer "B.Cu") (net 11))
 (segment (start 153.0225 83.1725) (end 151.275 81.8) (width 0.25) (layer "F.Cu") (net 12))
 (segment (start 154.45 89.318) (end 153.0225 87.8905) (width 0.25) (layer "F.Cu") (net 12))
 (segment (start 153.0225 87.8905) (end 153.0225 83.1725) (width 0.25) (layer "F.Cu") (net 12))
 (segment (start 151.275 81.8) (end 151.280657 77.274849) (width 0.25) (layer "F.Cu") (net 12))
 (segment (start 150.795522 74.645984) (end 150.825 76.225) (width 0.25) (layer "F.Cu") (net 13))
 (via (at 150.825 76.225) (size 0.8) (drill 0.4) (layers "F.Cu" "B.Cu") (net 13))
 (segment (start 151.91 76.98) (end 151.91 86.778) (width 0.25) (layer "B.Cu") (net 13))
 (segment (start 150.825 76.225) (end 151.91 76.98) (width 0.25) (layer "B.Cu") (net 13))
 (segment (start 150.272336 84.347336) (end 150.272336 77.274849) (width 0.25) (layer "F.Cu") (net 14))
 (segment (start 151.91 89.318) (end 150.6 88.008) (width 0.25) (layer "F.Cu") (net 14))
 (segment (start 150.6 84.675) (end 150.272336 84.347336) (width 0.25) (layer "F.Cu") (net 14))
 (segment (start 150.6 88.008) (end 150.6 84.675) (width 0.25) (layer "F.Cu") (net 14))
 (segment (start 149.809068 74.645984) (end 149.825 75.8) (width 0.25) (layer "F.Cu") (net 15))
 (via (at 149.825 75.8) (size 0.8) (drill 0.4) (layers "F.Cu" "B.Cu") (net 15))
 (segment (start 149.37 84.691) (end 149.37 86.778) (width 0.25) (layer "B.Cu") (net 15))
 (segment (start 149.825 84.05) (end 149.37 84.691) (width 0.25) (layer "B.Cu") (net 15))
 (segment (start 149.825 75.8) (end 149.825 84.05) (width 0.25) (layer "B.Cu") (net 15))
 (segment (start 147.9425 83.5785) (end 149.275 81.975) (width 0.25) (layer "F.Cu") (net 16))
 (segment (start 149.37 89.318) (end 147.9425 87.8905) (width 0.25) (layer "F.Cu") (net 16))
 (segment (start 149.275 81.975) (end 149.272114 77.270799) (width 0.25) (layer "F.Cu") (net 16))
 (segment (start 147.9425 87.8905) (end 147.9425 83.5785) (width 0.25) (layer "F.Cu") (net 16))
 (segment (start 148.825 76.225) (end 148.804183 74.639096) (width 0.25) (layer "F.Cu") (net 17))
 (via (at 148.825 76.225) (size 0.8) (drill 0.4) (layers "F.Cu" "B.Cu") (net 17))
 (segment (start 148.825 78.2) (end 146.83 79.738) (width 0.25) (layer "B.Cu") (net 17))
 (segment (start 146.83 79.738) (end 146.83 86.778) (width 0.25) (layer "B.Cu") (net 17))
 (segment (start 148.825 76.225) (end 148.825 78.2) (width 0.25) (layer "B.Cu") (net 17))
 (segment (start 145.7175 88.2055) (end 145.7175 83.3905) (width 0.25) (layer "F.Cu") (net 18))
 (segment (start 147.574 82.677) (end 148.25 81.875) (width 0.25) (layer "F.Cu") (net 18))
 (segment (start 146.431 82.677) (end 147.574 82.677) (width 0.25) (layer "F.Cu") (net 18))
 (segment (start 146.83 89.318) (end 145.7175 88.2055) (width 0.25) (layer "F.Cu") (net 18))
 (segment (start 145.7175 83.3905) (end 146.431 82.677) (width 0.25) (layer "F.Cu") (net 18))
 (segment (start 148.25 81.875) (end 148.267842 77.274849) (width 0.25) (layer "F.Cu") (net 18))
 (segment (start 147.79602 74.639096) (end 147.775 75.775) (width 0.25) (layer "F.Cu") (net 19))
 (via (at 147.775 75.775) (size 0.8) (drill 0.4) (layers "F.Cu" "B.Cu") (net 19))
 (segment (start 144.29 79.992) (end 144.29 86.778) (width 0.25) (layer "B.Cu") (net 19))
 (segment (start 147 78.232) (end 146.05 78.232) (width 0.25) (layer "B.Cu") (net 19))
 (segment (start 146.05 78.232) (end 144.29 79.992) (width 0.25) (layer "B.Cu") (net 19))
 (segment (start 147.775 75.775) (end 147.775 77.65) (width 0.25) (layer "B.Cu") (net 19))
 (segment (start 147.775 77.65) (end 147 78.232) (width 0.25) (layer "B.Cu") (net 19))
 (segment (start 144.29 89.318) (end 143.256 88.284) (width 0.25) (layer "F.Cu") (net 20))
 (segment (start 143.9 81.775) (end 146.775 81.775) (width 0.25) (layer "F.Cu") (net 20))
 (segment (start 143.256 88.284) (end 143.256 87.503) (width 0.25) (layer "F.Cu") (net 20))
 (segment (start 143.256 87.503) (end 143.1775 87.4245) (width 0.25) (layer "F.Cu") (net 20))
 (segment (start 143.1775 87.4245) (end 143.1775 82.6285) (width 0.25) (layer "F.Cu") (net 20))
 (segment (start 146.775 81.775) (end 147.275 81.125) (width 0.25) (layer "F.Cu") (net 20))
 (segment (start 147.275 81.125) (end 147.261007 77.269986) (width 0.25) (layer "F.Cu") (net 20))
 (segment (start 143.1775 82.6285) (end 143.9 81.775) (width 0.25) (layer "F.Cu") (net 20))
 (segment (start 146.800523 74.648349) (end 146.800523 76.199477) (width 0.25) (layer "F.Cu") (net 21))
 (segment (start 146.800523 76.199477) (end 146.8 76.2) (width 0.25) (layer "F.Cu") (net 21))
 (via (at 146.8 76.2) (size 0.8) (drill 0.4) (layers "F.Cu" "B.Cu") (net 21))
 (segment (start 141.75 79.738) (end 144.663 76.825) (width 0.25) (layer "B.Cu") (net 21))
 (segment (start 146.35 76.825) (end 146.8 76.2) (width 0.25) (layer "B.Cu") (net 21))
 (segment (start 141.75 86.778) (end 141.75 79.738) (width 0.25) (layer "B.Cu") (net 21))
 (segment (start 144.663 76.825) (end 146.35 76.825) (width 0.25) (layer "B.Cu") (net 21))
 (segment (start 141.75 89.318) (end 140.6375 88.2055) (width 0.25) (layer "F.Cu") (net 22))
 (segment (start 141.859 81.153) (end 145.669 81.153) (width 0.25) (layer "F.Cu") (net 22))
 (segment (start 140.6375 82.3745) (end 141.859 81.153) (width 0.25) (layer "F.Cu") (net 22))
 (segment (start 145.669 81.153) (end 146.275 80.625) (width 0.25) (layer "F.Cu") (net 22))
 (segment (start 140.6375 88.2055) (end 140.6375 82.3745) (width 0.25) (layer "F.Cu") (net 22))
 (segment (start 146.275 80.625) (end 146.269693 77.275817) (width 0.25) (layer "F.Cu") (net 22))
 (segment (start 145.80165 74.648349) (end 145.80165 75.74835) (width 0.25) (layer "F.Cu") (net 23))
 (segment (start 145.80165 75.74835) (end 145.8 75.75) (width 0.25) (layer "F.Cu") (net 23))
 (via (at 145.8 75.75) (size 0.8) (drill 0.4) (layers "F.Cu" "B.Cu") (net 23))
 (segment (start 145.35 76.2) (end 145.8 75.75) (width 0.25) (layer "B.Cu") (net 23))
 (segment (start 139.21 86.778) (end 139.21 78.214) (width 0.25) (layer "B.Cu") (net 23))
 (segment (start 139.21 78.214) (end 141.224 76.2) (width 0.25) (layer "B.Cu") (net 23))
 (segment (start 141.224 76.2) (end 145.35 76.2) (width 0.25) (layer "B.Cu") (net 23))
 (segment (start 142.35 79.4) (end 144.225 79.4) (width 0.25) (layer "F.Cu") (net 24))
 (segment (start 145.271167 78.221167) (end 145.271167 77.27545) (width 0.25) (layer "F.Cu") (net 24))
 (segment (start 137.795 83.955) (end 142.35 79.4) (width 0.25) (layer "F.Cu") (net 24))
 (segment (start 144.2 79.4) (end 145.275 78.225) (width 0.25) (layer "F.Cu") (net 24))
 (segment (start 139.21 89.318) (end 137.795 87.903) (width 0.25) (layer "F.Cu") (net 24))
 (segment (start 137.795 87.903) (end 137.795 83.955) (width 0.25) (layer "F.Cu") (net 24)))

